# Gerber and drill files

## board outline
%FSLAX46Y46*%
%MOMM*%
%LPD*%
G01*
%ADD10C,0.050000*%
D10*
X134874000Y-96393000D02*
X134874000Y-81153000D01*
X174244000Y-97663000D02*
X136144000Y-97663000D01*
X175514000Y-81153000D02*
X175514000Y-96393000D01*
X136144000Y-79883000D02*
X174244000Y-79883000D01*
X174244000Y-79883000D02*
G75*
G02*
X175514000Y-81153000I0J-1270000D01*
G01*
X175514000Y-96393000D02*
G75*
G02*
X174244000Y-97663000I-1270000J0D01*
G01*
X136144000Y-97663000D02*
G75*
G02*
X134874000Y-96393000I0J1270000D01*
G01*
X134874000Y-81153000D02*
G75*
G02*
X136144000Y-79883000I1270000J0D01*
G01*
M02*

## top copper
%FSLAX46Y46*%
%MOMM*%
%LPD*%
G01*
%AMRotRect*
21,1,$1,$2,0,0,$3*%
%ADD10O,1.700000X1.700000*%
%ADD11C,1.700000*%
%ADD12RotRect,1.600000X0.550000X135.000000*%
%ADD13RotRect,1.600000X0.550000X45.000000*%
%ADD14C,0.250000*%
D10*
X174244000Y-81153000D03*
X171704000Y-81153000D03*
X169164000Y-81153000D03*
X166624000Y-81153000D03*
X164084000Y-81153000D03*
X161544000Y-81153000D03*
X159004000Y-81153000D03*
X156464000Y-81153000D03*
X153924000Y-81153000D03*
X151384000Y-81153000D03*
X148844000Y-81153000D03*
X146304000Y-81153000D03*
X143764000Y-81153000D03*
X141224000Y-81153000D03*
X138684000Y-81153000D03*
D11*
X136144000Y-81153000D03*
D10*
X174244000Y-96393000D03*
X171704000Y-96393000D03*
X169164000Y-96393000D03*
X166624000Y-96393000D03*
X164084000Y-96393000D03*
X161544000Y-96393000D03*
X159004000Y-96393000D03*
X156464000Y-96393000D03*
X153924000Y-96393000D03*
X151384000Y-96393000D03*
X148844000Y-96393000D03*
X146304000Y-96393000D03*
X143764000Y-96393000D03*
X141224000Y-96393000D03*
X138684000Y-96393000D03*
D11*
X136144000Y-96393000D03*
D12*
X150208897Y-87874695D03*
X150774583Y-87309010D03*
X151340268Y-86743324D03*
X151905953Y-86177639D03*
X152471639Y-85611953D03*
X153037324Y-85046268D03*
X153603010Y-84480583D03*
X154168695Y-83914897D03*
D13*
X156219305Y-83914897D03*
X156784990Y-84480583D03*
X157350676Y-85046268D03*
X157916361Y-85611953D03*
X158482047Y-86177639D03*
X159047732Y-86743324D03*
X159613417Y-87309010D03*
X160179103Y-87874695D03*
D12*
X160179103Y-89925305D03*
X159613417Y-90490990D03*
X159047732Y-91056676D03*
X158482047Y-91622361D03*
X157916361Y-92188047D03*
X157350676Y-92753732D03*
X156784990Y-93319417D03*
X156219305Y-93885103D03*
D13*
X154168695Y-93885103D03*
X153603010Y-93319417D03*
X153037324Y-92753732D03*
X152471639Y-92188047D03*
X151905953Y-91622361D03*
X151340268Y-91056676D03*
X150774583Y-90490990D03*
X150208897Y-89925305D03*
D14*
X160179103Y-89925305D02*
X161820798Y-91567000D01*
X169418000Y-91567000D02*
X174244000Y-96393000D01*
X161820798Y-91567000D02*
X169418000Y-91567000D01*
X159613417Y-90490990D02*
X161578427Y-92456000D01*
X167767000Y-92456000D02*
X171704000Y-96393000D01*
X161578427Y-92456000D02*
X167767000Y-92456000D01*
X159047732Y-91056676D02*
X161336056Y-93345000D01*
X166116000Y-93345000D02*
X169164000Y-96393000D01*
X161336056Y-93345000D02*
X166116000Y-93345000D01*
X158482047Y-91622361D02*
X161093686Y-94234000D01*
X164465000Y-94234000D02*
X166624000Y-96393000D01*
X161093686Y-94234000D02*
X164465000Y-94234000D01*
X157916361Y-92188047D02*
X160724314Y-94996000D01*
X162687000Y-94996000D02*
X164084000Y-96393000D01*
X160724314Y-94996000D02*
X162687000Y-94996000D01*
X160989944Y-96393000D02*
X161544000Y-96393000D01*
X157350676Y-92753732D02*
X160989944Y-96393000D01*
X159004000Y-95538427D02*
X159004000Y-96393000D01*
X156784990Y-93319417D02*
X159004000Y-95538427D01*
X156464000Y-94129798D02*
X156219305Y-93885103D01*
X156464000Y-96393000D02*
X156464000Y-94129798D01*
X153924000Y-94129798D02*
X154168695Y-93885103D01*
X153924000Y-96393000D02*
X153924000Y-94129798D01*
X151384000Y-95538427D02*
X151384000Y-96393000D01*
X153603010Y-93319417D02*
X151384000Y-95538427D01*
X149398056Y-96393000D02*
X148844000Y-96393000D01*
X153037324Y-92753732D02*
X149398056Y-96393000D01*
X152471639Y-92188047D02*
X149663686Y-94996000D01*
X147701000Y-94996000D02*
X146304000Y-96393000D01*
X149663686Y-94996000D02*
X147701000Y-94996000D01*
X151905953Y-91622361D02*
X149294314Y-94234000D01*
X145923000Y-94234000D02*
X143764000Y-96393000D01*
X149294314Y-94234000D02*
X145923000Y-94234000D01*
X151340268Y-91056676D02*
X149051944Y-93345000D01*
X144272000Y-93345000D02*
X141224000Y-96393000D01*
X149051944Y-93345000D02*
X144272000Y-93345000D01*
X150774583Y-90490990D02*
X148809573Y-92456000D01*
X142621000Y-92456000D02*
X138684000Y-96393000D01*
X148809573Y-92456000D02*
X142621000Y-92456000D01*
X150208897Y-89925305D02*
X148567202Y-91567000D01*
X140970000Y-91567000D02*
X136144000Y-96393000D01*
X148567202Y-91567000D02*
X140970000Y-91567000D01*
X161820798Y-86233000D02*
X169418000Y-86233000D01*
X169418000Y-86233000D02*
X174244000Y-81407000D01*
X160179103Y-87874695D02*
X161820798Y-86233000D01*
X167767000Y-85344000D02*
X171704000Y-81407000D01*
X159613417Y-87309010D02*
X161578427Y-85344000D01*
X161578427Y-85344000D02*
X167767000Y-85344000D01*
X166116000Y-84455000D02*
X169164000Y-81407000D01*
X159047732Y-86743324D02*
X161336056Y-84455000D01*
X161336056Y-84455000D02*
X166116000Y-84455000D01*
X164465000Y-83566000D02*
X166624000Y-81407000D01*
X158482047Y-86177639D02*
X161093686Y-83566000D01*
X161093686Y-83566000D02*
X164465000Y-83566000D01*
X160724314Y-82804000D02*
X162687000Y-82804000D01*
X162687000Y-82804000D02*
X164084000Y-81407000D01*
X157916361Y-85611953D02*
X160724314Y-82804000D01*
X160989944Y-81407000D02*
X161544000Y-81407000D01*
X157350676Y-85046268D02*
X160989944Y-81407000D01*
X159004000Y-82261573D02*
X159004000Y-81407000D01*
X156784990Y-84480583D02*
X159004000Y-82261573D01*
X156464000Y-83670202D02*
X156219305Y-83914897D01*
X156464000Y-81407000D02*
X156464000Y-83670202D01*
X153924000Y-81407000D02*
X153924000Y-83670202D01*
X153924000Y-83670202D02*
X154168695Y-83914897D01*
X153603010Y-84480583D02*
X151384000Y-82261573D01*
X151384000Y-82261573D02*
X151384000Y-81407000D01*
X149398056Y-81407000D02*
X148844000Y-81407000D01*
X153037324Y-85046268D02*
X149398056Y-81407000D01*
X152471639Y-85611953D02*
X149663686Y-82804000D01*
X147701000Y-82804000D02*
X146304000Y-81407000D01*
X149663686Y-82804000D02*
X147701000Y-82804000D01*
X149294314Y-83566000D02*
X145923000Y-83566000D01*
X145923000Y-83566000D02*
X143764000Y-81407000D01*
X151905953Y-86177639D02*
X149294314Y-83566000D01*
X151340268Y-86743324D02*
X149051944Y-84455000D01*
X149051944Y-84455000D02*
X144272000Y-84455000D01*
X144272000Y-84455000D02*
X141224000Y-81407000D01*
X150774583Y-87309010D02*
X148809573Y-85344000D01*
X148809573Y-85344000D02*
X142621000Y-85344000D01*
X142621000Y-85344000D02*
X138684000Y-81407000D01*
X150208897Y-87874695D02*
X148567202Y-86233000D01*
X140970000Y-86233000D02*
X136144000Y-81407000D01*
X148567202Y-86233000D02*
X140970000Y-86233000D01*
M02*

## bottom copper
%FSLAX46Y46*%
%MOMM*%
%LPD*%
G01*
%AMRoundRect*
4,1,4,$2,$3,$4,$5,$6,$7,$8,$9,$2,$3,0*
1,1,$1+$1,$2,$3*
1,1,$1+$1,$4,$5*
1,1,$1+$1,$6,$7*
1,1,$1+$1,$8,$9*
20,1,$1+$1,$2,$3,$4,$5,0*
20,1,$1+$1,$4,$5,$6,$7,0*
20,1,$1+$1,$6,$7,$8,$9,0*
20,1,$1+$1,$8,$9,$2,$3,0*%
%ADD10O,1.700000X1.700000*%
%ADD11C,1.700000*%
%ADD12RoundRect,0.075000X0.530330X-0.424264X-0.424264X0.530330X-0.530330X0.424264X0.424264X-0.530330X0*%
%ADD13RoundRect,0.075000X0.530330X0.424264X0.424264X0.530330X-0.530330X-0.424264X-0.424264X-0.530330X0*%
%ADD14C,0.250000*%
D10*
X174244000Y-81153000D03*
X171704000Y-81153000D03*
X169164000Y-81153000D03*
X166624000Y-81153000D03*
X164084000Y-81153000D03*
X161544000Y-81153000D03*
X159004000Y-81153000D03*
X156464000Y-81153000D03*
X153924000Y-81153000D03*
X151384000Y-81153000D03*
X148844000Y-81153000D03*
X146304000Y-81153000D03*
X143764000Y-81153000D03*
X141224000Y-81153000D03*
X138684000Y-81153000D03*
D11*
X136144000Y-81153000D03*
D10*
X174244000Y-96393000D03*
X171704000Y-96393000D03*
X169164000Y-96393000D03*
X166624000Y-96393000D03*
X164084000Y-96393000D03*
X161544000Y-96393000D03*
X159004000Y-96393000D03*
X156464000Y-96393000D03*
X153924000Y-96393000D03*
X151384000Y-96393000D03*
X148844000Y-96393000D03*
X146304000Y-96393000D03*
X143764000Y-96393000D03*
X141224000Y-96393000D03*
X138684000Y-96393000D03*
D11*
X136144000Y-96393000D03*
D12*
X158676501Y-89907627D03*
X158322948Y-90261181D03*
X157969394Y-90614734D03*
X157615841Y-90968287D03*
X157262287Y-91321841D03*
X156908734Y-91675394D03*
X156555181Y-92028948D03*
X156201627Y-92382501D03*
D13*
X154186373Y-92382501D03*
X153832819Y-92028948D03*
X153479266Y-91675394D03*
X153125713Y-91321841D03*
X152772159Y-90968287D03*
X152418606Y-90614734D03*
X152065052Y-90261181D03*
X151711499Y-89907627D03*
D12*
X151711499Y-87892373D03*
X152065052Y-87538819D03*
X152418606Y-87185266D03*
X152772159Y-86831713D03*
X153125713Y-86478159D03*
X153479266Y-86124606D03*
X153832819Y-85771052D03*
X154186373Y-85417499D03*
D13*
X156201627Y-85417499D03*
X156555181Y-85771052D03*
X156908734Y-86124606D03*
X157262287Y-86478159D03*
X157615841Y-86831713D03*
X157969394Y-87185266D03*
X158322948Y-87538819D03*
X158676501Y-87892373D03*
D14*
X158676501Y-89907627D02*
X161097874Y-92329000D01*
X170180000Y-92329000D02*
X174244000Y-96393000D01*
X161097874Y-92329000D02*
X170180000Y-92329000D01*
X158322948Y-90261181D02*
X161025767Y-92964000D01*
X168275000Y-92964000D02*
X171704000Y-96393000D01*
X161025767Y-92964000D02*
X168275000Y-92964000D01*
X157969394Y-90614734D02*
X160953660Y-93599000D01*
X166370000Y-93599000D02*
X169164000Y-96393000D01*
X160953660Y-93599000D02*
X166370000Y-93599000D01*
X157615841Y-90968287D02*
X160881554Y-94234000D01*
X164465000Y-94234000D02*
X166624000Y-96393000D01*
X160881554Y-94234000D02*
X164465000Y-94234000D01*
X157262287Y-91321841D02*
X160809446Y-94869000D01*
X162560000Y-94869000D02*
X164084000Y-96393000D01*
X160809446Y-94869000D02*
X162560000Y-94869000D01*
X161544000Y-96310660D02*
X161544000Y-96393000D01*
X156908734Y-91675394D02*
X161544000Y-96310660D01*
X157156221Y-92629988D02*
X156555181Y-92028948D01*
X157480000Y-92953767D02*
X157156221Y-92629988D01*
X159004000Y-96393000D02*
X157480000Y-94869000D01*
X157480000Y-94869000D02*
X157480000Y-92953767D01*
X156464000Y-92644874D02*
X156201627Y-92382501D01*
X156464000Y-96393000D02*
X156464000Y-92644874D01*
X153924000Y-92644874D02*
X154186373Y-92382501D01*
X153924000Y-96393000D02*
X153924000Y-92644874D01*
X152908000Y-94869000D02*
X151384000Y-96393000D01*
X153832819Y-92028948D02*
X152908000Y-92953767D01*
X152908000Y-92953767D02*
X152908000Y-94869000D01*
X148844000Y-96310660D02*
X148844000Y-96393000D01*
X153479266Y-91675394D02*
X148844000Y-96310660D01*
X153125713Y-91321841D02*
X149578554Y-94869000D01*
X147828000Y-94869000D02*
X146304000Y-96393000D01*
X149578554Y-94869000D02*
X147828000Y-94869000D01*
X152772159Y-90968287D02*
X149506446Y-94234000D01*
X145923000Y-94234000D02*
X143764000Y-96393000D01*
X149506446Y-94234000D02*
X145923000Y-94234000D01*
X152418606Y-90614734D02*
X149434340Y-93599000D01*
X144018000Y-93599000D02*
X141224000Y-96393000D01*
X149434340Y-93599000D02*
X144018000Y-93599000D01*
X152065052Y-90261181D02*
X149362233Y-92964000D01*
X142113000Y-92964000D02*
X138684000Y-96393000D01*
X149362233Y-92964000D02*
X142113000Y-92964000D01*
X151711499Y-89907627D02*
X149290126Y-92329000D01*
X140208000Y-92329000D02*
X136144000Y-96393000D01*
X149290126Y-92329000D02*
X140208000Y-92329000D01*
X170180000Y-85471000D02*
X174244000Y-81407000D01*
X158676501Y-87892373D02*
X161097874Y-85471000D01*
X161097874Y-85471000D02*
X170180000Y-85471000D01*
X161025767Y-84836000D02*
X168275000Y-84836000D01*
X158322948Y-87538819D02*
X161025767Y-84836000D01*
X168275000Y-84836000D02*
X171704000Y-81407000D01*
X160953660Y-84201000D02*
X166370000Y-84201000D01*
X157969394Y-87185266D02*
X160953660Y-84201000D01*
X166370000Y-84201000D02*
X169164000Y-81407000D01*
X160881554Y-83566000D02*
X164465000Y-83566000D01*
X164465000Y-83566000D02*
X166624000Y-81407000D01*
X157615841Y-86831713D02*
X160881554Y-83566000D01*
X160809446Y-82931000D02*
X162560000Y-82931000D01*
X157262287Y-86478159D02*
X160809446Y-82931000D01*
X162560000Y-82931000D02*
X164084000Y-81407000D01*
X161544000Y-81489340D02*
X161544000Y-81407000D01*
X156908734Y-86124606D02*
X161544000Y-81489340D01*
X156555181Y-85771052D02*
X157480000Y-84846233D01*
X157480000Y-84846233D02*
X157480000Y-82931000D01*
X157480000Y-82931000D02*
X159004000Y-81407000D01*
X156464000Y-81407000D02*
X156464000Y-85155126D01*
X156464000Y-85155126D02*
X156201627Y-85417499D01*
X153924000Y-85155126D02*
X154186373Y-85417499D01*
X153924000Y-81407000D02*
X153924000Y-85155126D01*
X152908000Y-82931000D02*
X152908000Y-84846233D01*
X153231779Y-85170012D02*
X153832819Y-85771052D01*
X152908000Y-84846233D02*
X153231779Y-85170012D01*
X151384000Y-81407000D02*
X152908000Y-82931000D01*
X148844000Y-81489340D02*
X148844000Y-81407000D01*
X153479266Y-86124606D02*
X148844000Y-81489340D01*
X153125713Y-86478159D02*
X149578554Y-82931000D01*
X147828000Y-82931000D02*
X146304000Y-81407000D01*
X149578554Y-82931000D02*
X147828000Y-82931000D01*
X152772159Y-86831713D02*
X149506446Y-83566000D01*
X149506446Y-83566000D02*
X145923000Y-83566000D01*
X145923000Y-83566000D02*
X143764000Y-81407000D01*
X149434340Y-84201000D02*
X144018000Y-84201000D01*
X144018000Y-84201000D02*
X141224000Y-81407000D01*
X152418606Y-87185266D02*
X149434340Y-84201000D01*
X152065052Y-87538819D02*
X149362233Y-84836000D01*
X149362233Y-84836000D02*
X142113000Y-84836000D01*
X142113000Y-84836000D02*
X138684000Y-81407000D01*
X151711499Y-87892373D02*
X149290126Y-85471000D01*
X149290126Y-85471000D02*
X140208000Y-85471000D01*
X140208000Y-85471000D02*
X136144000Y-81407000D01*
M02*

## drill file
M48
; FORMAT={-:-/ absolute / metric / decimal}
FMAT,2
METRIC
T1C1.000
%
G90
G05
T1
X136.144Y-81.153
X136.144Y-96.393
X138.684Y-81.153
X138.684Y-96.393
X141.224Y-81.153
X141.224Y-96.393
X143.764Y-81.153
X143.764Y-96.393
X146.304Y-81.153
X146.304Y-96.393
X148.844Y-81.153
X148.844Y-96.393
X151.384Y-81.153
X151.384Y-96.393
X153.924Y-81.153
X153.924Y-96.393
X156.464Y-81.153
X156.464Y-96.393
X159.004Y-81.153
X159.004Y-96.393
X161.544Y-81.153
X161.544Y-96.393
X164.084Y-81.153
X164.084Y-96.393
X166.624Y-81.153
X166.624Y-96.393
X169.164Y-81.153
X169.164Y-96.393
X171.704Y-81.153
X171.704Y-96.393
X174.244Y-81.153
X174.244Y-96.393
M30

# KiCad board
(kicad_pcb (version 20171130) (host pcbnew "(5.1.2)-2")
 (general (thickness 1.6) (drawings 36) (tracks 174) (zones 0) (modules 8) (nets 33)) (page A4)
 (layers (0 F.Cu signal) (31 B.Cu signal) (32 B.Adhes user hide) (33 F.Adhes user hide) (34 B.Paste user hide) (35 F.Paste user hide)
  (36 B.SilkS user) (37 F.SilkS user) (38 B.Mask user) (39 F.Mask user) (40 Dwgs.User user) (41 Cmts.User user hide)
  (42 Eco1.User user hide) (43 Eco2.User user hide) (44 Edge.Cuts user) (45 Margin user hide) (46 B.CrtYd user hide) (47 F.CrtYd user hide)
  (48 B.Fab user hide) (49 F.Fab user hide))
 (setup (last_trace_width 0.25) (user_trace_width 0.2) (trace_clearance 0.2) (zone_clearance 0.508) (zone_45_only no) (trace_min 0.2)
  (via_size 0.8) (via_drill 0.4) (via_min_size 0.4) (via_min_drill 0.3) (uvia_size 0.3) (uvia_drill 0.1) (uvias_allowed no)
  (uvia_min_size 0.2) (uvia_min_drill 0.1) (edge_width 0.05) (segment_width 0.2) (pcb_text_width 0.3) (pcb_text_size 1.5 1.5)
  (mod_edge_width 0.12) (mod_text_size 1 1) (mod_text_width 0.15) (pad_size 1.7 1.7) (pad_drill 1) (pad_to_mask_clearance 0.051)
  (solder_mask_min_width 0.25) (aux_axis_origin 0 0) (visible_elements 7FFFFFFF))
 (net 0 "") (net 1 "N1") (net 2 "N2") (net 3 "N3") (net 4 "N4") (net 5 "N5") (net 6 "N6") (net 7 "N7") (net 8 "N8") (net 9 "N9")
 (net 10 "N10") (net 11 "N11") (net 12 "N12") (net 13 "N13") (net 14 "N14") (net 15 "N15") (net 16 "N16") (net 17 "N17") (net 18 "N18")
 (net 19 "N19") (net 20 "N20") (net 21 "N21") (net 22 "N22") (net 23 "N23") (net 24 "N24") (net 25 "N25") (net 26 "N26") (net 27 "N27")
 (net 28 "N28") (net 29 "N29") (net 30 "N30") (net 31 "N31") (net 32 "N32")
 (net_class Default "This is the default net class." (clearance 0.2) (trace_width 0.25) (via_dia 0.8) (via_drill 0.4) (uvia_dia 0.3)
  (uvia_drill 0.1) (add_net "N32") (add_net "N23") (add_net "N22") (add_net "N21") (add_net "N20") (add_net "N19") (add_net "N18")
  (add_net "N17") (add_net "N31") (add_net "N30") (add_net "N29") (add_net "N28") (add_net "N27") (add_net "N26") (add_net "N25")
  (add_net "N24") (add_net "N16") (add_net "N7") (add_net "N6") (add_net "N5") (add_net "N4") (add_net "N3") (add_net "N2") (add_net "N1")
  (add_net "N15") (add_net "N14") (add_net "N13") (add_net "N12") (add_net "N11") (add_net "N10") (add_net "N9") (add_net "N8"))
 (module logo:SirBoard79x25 (layer B.Cu) (at 169.164 93.599 180)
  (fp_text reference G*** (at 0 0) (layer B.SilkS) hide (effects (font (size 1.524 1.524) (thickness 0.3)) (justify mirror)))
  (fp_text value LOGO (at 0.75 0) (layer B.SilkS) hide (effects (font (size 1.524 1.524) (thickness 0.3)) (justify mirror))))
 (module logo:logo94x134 (layer B.Cu) (at 169.164 87.122 180)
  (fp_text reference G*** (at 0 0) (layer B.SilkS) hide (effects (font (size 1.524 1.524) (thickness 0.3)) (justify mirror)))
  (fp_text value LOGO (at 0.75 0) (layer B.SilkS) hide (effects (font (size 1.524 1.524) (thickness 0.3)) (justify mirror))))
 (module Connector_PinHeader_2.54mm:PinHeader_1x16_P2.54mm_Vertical (layer B.Cu) (at 136.144 81.153 270)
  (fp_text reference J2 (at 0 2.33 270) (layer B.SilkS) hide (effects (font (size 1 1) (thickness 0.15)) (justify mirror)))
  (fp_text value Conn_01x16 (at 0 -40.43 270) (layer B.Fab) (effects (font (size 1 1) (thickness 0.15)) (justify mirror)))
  (pad 16 thru_hole oval (at 0 -38.1 270) (size 1.7 1.7) (drill 1) (layers *.Cu *.Mask) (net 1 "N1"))
  (pad 15 thru_hole oval (at 0 -35.56 270) (size 1.7 1.7) (drill 1) (layers *.Cu *.Mask) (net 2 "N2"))
  (pad 14 thru_hole oval (at 0 -33.02 270) (size 1.7 1.7) (drill 1) (layers *.Cu *.Mask) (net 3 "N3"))
  (pad 13 thru_hole oval (at 0 -30.48 270) (size 1.7 1.7) (drill 1) (layers *.Cu *.Mask) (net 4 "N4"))
  (pad 12 thru_hole oval (at 0 -27.94 270) (size 1.7 1.7) (drill 1) (layers *.Cu *.Mask) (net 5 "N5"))
  (pad 11 thru_hole oval (at 0 -25.4 270) (size 1.7 1.7) (drill 1) (layers *.Cu *.Mask) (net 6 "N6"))
  (pad 10 thru_hole oval (at 0 -22.86 270) (size 1.7 1.7) (drill 1) (layers *.Cu *.Mask) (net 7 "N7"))
  (pad 9 thru_hole oval (at 0 -20.32 270) (size 1.7 1.7) (drill 1) (layers *.Cu *.Mask) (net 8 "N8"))
  (pad 8 thru_hole oval (at 0 -17.78 270) (size 1.7 1.7) (drill 1) (layers *.Cu *.Mask) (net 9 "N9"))
  (pad 7 thru_hole oval (at 0 -15.24 270) (size 1.7 1.7) (drill 1) (layers *.Cu *.Mask) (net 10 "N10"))
  (pad 6 thru_hole oval (at 0 -12.7 270) (size 1.7 1.7) (drill 1) (layers *.Cu *.Mask) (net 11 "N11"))
  (pad 5 thru_hole oval (at 0 -10.16 270) (size 1.7 1.7) (drill 1) (layers *.Cu *.Mask) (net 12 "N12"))
  (pad 4 thru_hole oval (at 0 -7.62 270) (size 1.7 1.7) (drill 1) (layers *.Cu *.Mask) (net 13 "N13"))
  (pad 3 thru_hole oval (at 0 -5.08 270) (size 1.7 1.7) (drill 1) (layers *.Cu *.Mask) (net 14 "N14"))
  (pad 2 thru_hole oval (at 0 -2.54 270) (size 1.7 1.7) (drill 1) (layers *.Cu *.Mask) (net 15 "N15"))
  (pad 1 thru_hole circle (at 0 0 270) (size 1.7 1.7) (drill 1) (layers *.Cu *.Mask) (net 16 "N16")))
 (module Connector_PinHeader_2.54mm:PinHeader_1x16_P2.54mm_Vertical (layer B.Cu) (at 136.144 96.393 270)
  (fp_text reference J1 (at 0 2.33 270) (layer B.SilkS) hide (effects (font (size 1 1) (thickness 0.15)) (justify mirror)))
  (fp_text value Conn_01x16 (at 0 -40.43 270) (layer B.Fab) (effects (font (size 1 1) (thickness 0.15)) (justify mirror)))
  (pad 16 thru_hole oval (at 0 -38.1 270) (size 1.7 1.7) (drill 1) (layers *.Cu *.Mask) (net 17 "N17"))
  (pad 15 thru_hole oval (at 0 -35.56 270) (size 1.7 1.7) (drill 1) (layers *.Cu *.Mask) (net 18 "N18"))
  (pad 14 thru_hole oval (at 0 -33.02 270) (size 1.7 1.7) (drill 1) (layers *.Cu *.Mask) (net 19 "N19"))
  (pad 13 thru_hole oval (at 0 -30.48 270) (size 1.7 1.7) (drill 1) (layers *.Cu *.Mask) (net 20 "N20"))
  (pad 12 thru_hole oval (at 0 -27.94 270) (size 1.7 1.7) (drill 1) (layers *.Cu *.Mask) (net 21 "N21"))
  (pad 11 thru_hole oval (at 0 -25.4 270) (size 1.7 1.7) (drill 1) (layers *.Cu *.Mask) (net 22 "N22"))
  (pad 10 thru_hole oval (at 0 -22.86 270) (size 1.7 1.7) (drill 1) (layers *.Cu *.Mask) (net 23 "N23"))
  (pad 9 thru_hole oval (at 0 -20.32 270) (size 1.7 1.7) (drill 1) (layers *.Cu *.Mask) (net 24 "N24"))
  (pad 8 thru_hole oval (at 0 -17.78 270) (size 1.7 1.7) (drill 1) (layers *.Cu *.Mask) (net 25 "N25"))
  (pad 7 thru_hole oval (at 0 -15.24 270) (size 1.7 1.7) (drill 1) (layers *.Cu *.Mask) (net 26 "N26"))
  (pad 6 thru_hole oval (at 0 -12.7 270) (size 1.7 1.7) (drill 1) (layers *.Cu *.Mask) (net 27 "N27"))
  (pad 5 thru_hole oval (at 0 -10.16 270) (size 1.7 1.7) (drill 1) (layers *.Cu *.Mask) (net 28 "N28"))
  (pad 4 thru_hole oval (at 0 -7.62 270) (size 1.7 1.7) (drill 1) (layers *.Cu *.Mask) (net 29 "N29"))
  (pad 3 thru_hole oval (at 0 -5.08 270) (size 1.7 1.7) (drill 1) (layers *.Cu *.Mask) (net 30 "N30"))
  (pad 2 thru_hole oval (at 0 -2.54 270) (size 1.7 1.7) (drill 1) (layers *.Cu *.Mask) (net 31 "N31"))
  (pad 1 thru_hole circle (at 0 0 270) (size 1.7 1.7) (drill 1) (layers *.Cu *.Mask) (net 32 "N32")))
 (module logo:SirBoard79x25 (layer F.Cu) (at 141.224 93.726)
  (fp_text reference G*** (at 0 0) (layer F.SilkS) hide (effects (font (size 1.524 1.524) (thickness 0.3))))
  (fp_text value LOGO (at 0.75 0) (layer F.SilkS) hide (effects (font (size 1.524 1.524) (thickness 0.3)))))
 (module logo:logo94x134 (layer F.Cu) (at 141.224 87.249)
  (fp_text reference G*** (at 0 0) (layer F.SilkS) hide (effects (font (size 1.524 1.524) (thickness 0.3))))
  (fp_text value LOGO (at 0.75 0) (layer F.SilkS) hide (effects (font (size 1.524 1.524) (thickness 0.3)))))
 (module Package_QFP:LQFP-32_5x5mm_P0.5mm (layer B.Cu) (at 155.194 88.9 135)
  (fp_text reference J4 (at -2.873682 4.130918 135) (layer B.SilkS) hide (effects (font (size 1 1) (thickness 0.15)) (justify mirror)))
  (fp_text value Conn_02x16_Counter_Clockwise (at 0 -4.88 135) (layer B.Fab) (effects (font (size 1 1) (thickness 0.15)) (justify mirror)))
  (pad 1 smd roundrect (at -3.175 1.75 135) (size 1.5 0.3) (layers B.Cu B.Paste B.Mask) (roundrect_rratio 0.25) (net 17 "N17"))
  (pad 2 smd roundrect (at -3.175 1.25 135) (size 1.5 0.3) (layers B.Cu B.Paste B.Mask) (roundrect_rratio 0.25) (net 18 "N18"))
  (pad 3 smd roundrect (at -3.175 0.75 135) (size 1.5 0.3) (layers B.Cu B.Paste B.Mask) (roundrect_rratio 0.25) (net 19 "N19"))
  (pad 4 smd roundrect (at -3.175 0.25 135) (size 1.5 0.3) (layers B.Cu B.Paste B.Mask) (roundrect_rratio 0.25) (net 20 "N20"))
  (pad 5 smd roundrect (at -3.175 -0.25 135) (size 1.5 0.3) (layers B.Cu B.Paste B.Mask) (roundrect_rratio 0.25) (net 21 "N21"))
  (pad 6 smd roundrect (at -3.175 -0.75 135) (size 1.5 0.3) (layers B.Cu B.Paste B.Mask) (roundrect_rratio 0.25) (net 22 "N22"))
  (pad 7 smd roundrect (at -3.175 -1.25 135) (size 1.5 0.3) (layers B.Cu B.Paste B.Mask) (roundrect_rratio 0.25) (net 23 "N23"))
  (pad 8 smd roundrect (at -3.175 -1.75 135) (size 1.5 0.3) (layers B.Cu B.Paste B.Mask) (roundrect_rratio 0.25) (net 24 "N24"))
  (pad 9 smd roundrect (at -1.75 -3.175 135) (size 0.3 1.5) (layers B.Cu B.Paste B.Mask) (roundrect_rratio 0.25) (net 25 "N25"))
  (pad 10 smd roundrect (at -1.25 -3.175 135) (size 0.3 1.5) (layers B.Cu B.Paste B.Mask) (roundrect_rratio 0.25) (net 26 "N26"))
  (pad 11 smd roundrect (at -0.75 -3.175 135) (size 0.3 1.5) (layers B.Cu B.Paste B.Mask) (roundrect_rratio 0.25) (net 27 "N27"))
  (pad 12 smd roundrect (at -0.25 -3.175 135) (size 0.3 1.5) (layers B.Cu B.Paste B.Mask) (roundrect_rratio 0.25) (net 28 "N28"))
  (pad 13 smd roundrect (at 0.25 -3.175 135) (size 0.3 1.5) (layers B.Cu B.Paste B.Mask) (roundrect_rratio 0.25) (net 29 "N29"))
  (pad 14 smd roundrect (at 0.75 -3.175 135) (size 0.3 1.5) (layers B.Cu B.Paste B.Mask) (roundrect_rratio 0.25) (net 30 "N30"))
  (pad 15 smd roundrect (at 1.25 -3.175 135) (size 0.3 1.5) (layers B.Cu B.Paste B.Mask) (roundrect_rratio 0.25) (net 31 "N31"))
  (pad 16 smd roundrect (at 1.75 -3.175 135) (size 0.3 1.5) (layers B.Cu B.Paste B.Mask) (roundrect_rratio 0.25) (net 32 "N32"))
  (pad 17 smd roundrect (at 3.175 -1.75 135) (size 1.5 0.3) (layers B.Cu B.Paste B.Mask) (roundrect_rratio 0.25) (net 16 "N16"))
  (pad 18 smd roundrect (at 3.175 -1.25 135) (size 1.5 0.3) (layers B.Cu B.Paste B.Mask) (roundrect_rratio 0.25) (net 15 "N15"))
  (pad 19 smd roundrect (at 3.175 -0.75 135) (size 1.5 0.3) (layers B.Cu B.Paste B.Mask) (roundrect_rratio 0.25) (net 14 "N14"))
  (pad 20 smd roundrect (at 3.175 -0.25 135) (size 1.5 0.3) (layers B.Cu B.Paste B.Mask) (roundrect_rratio 0.25) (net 13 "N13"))
  (pad 21 smd roundrect (at 3.175 0.25 135) (size 1.5 0.3) (layers B.Cu B.Paste B.Mask) (roundrect_rratio 0.25) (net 12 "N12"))
  (pad 22 smd roundrect (at 3.175 0.75 135) (size 1.5 0.3) (layers B.Cu B.Paste B.Mask) (roundrect_rratio 0.25) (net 11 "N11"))
  (pad 23 smd roundrect (at 3.175 1.25 135) (size 1.5 0.3) (layers B.Cu B.Paste B.Mask) (roundrect_rratio 0.25) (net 10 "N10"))
  (pad 24 smd roundrect (at 3.175 1.75 135) (size 1.5 0.3) (layers B.Cu B.Paste B.Mask) (roundrect_rratio 0.25) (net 9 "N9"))
  (pad 25 smd roundrect (at 1.75 3.175 135) (size 0.3 1.5) (layers B.Cu B.Paste B.Mask) (roundrect_rratio 0.25) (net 8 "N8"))
  (pad 26 smd roundrect (at 1.25 3.175 135) (size 0.3 1.5) (layers B.Cu B.Paste B.Mask) (roundrect_rratio 0.25) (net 7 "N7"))
  (pad 27 smd roundrect (at 0.75 3.175 135) (size 0.3 1.5) (layers B.Cu B.Paste B.Mask) (roundrect_rratio 0.25) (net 6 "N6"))
  (pad 28 smd roundrect (at 0.25 3.175 135) (size 0.3 1.5) (layers B.Cu B.Paste B.Mask) (roundrect_rratio 0.25) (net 5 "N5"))
  (pad 29 smd roundrect (at -0.25 3.175 135) (size 0.3 1.5) (layers B.Cu B.Paste B.Mask) (roundrect_rratio 0.25) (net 4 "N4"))
  (pad 30 smd roundrect (at -0.75 3.175 135) (size 0.3 1.5) (layers B.Cu B.Paste B.Mask) (roundrect_rratio 0.25) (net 3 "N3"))
  (pad 31 smd roundrect (at -1.25 3.175 135) (size 0.3 1.5) (layers B.Cu B.Paste B.Mask) (roundrect_rratio 0.25) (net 2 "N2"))
  (pad 32 smd roundrect (at -1.75 3.175 135) (size 0.3 1.5) (layers B.Cu B.Paste B.Mask) (roundrect_rratio 0.25) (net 1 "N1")))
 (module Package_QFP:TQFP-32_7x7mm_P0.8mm (layer F.Cu) (at 155.194 88.9 45)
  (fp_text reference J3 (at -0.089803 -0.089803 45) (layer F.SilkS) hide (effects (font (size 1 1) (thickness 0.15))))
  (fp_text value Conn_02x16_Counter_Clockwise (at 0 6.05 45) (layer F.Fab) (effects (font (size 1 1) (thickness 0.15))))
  (pad 32 smd rect (at -2.8 -4.25 135) (size 1.6 0.55) (layers F.Cu F.Paste F.Mask) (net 16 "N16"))
  (pad 31 smd rect (at -2 -4.25 135) (size 1.6 0.55) (layers F.Cu F.Paste F.Mask) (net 15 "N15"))
  (pad 30 smd rect (at -1.2 -4.25 135) (size 1.6 0.55) (layers F.Cu F.Paste F.Mask) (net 14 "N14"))
  (pad 29 smd rect (at -0.4 -4.25 135) (size 1.6 0.55) (layers F.Cu F.Paste F.Mask) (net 13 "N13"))
  (pad 28 smd rect (at 0.4 -4.25 135) (size 1.6 0.55) (layers F.Cu F.Paste F.Mask) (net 12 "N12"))
  (pad 27 smd rect (at 1.2 -4.25 135) (size 1.6 0.55) (layers F.Cu F.Paste F.Mask) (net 11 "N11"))
  (pad 26 smd rect (at 2 -4.25 135) (size 1.6 0.55) (layers F.Cu F.Paste F.Mask) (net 10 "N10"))
  (pad 25 smd rect (at 2.8 -4.25 135) (size 1.6 0.55) (layers F.Cu F.Paste F.Mask) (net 9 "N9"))
  (pad 24 smd rect (at 4.25 -2.8 45) (size 1.6 0.55) (layers F.Cu F.Paste F.Mask) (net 8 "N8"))
  (pad 23 smd rect (at 4.25 -2 45) (size 1.6 0.55) (layers F.Cu F.Paste F.Mask) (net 7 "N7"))
  (pad 22 smd rect (at 4.25 -1.2 45) (size 1.6 0.55) (layers F.Cu F.Paste F.Mask) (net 6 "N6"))
  (pad 21 smd rect (at 4.25 -0.4 45) (size 1.6 0.55) (layers F.Cu F.Paste F.Mask) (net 5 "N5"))
  (pad 20 smd rect (at 4.25 0.4 45) (size 1.6 0.55) (layers F.Cu F.Paste F.Mask) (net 4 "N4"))
  (pad 19 smd rect (at 4.25 1.2 45) (size 1.6 0.55) (layers F.Cu F.Paste F.Mask) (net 3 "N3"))
  (pad 18 smd rect (at 4.25 2 45) (size 1.6 0.55) (layers F.Cu F.Paste F.Mask) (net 2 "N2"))
  (pad 17 smd rect (at 4.25 2.8 45) (size 1.6 0.55) (layers F.Cu F.Paste F.Mask) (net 1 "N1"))
  (pad 16 smd rect (at 2.8 4.25 135) (size 1.6 0.55) (layers F.Cu F.Paste F.Mask) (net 17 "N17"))
  (pad 15 smd rect (at 2 4.25 135) (size 1.6 0.55) (layers F.Cu F.Paste F.Mask) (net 18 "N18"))
  (pad 14 smd rect (at 1.2 4.25 135) (size 1.6 0.55) (layers F.Cu F.Paste F.Mask) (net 19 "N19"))
  (pad 13 smd rect (at 0.4 4.25 135) (size 1.6 0.55) (layers F.Cu F.Paste F.Mask) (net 20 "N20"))
  (pad 12 smd rect (at -0.4 4.25 135) (size 1.6 0.55) (layers F.Cu F.Paste F.Mask) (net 21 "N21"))
  (pad 11 smd rect (at -1.2 4.25 135) (size 1.6 0.55) (layers F.Cu F.Paste F.Mask) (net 22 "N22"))
  (pad 10 smd rect (at -2 4.25 135) (size 1.6 0.55) (layers F.Cu F.Paste F.Mask) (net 23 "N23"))
  (pad 9 smd rect (at -2.8 4.25 135) (size 1.6 0.55) (layers F.Cu F.Paste F.Mask) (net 24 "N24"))
  (pad 8 smd rect (at -4.25 2.8 45) (size 1.6 0.55) (layers F.Cu F.Paste F.Mask) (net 25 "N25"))
  (pad 7 smd rect (at -4.25 2 45) (size 1.6 0.55) (layers F.Cu F.Paste F.Mask) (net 26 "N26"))
  (pad 6 smd rect (at -4.25 1.2 45) (size 1.6 0.55) (layers F.Cu F.Paste F.Mask) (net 27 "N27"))
  (pad 5 smd rect (at -4.25 0.4 45) (size 1.6 0.55) (layers F.Cu F.Paste F.Mask) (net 28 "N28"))
  (pad 4 smd rect (at -4.25 -0.4 45) (size 1.6 0.55) (layers F.Cu F.Paste F.Mask) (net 29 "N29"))
  (pad 3 smd rect (at -4.25 -1.2 45) (size 1.6 0.55) (layers F.Cu F.Paste F.Mask) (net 30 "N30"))
  (pad 2 smd rect (at -4.25 -2 45) (size 1.6 0.55) (layers F.Cu F.Paste F.Mask) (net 31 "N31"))
  (pad 1 smd rect (at -4.25 -2.8 45) (size 1.6 0.55) (layers F.Cu F.Paste F.Mask) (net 32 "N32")))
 (gr_line (start 134.874 96.393) (end 134.874 81.153) (layer Edge.Cuts) (width 0.05))
 (gr_line (start 174.244 97.663) (end 136.144 97.663) (layer Edge.Cuts) (width 0.05))
 (gr_line (start 175.514 81.153) (end 175.514 96.393) (layer Edge.Cuts) (width 0.05))
 (gr_line (start 136.144 79.883) (end 174.244 79.883) (layer Edge.Cuts) (width 0.05))
 (gr_arc (start 174.244 81.153) (end 175.514 81.153) (angle -90) (layer Edge.Cuts) (width 0.05))
 (gr_arc (start 174.244 96.393) (end 174.244 97.663) (angle -90) (layer Edge.Cuts) (width 0.05))
 (gr_arc (start 136.144 96.393) (end 134.874 96.393) (angle -90) (layer Edge.Cuts) (width 0.05))
 (gr_arc (start 136.144 81.153) (end 136.144 79.883) (angle -90) (layer Edge.Cuts) (width 0.05))
 (segment (start 160.179103 89.925305) (end 161.820798 91.567) (width 0.25) (layer F.Cu) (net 17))
 (segment (start 169.418 91.567) (end 174.244 96.393) (width 0.25) (layer F.Cu) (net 17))
 (segment (start 161.820798 91.567) (end 169.418 91.567) (width 0.25) (layer F.Cu) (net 17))
 (segment (start 158.676501 89.907627) (end 161.097874 92.329) (width 0.25) (layer B.Cu) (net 17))
 (segment (start 170.18 92.329) (end 174.244 96.393) (width 0.25) (layer B.Cu) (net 17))
 (segment (start 161.097874 92.329) (end 170.18 92.329) (width 0.25) (layer B.Cu) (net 17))
 (segment (start 159.613417 90.49099) (end 161.578427 92.456) (width 0.25) (layer F.Cu) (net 18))
 (segment (start 167.767 92.456) (end 171.704 96.393) (width 0.25) (layer F.Cu) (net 18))
 (segment (start 161.578427 92.456) (end 167.767 92.456) (width 0.25) (layer F.Cu) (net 18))
 (segment (start 158.322948 90.261181) (end 161.025767 92.964) (width 0.25) (layer B.Cu) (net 18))
 (segment (start 168.275 92.964) (end 171.704 96.393) (width 0.25) (layer B.Cu) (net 18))
 (segment (start 161.025767 92.964) (end 168.275 92.964) (width 0.25) (layer B.Cu) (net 18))
 (segment (start 159.047732 91.056676) (end 161.336056 93.345) (width 0.25) (layer F.Cu) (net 19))
 (segment (start 166.116 93.345) (end 169.164 96.393) (width 0.25) (layer F.Cu) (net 19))
 (segment (start 161.336056 93.345) (end 166.116 93.345) (width 0.25) (layer F.Cu) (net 19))
 (segment (start 157.969394 90.614734) (end 160.95366 93.599) (width 0.25) (layer B.Cu) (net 19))
 (segment (start 166.37 93.599) (end 169.164 96.393) (width 0.25) (layer B.Cu) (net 19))
 (segment (start 160.95366 93.599) (end 166.37 93.599) (width 0.25) (layer B.Cu) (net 19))
 (segment (start 158.482047 91.622361) (end 161.093686 94.234) (width 0.25) (layer F.Cu) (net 20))
 (segment (start 164.465 94.234) (end 166.624 96.393) (width 0.25) (layer F.Cu) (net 20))
 (segment (start 161.093686 94.234) (end 164.465 94.234) (width 0.25) (layer F.Cu) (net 20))
 (segment (start 157.615841 90.968287) (end 160.881554 94.234) (width 0.25) (layer B.Cu) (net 20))
 (segment (start 164.465 94.234) (end 166.624 96.393) (width 0.25) (layer B.Cu) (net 20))
 (segment (start 160.881554 94.234) (end 164.465 94.234) (width 0.25) (layer B.Cu) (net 20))
 (segment (start 157.916361 92.188047) (end 160.724314 94.996) (width 0.25) (layer F.Cu) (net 21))
 (segment (start 162.687 94.996) (end 164.084 96.393) (width 0.25) (layer F.Cu) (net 21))
 (segment (start 160.724314 94.996) (end 162.687 94.996) (width 0.25) (layer F.Cu) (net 21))
 (segment (start 157.262287 91.321841) (end 160.809446 94.869) (width 0.25) (layer B.Cu) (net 21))
 (segment (start 162.56 94.869) (end 164.084 96.393) (width 0.25) (layer B.Cu) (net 21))
 (segment (start 160.809446 94.869) (end 162.56 94.869) (width 0.25) (layer B.Cu) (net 21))
 (segment (start 160.989944 96.393) (end 161.544 96.393) (width 0.25) (layer F.Cu) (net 22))
 (segment (start 157.350676 92.753732) (end 160.989944 96.393) (width 0.25) (layer F.Cu) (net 22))
 (segment (start 161.544 96.31066) (end 161.544 96.393) (width 0.25) (layer B.Cu) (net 22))
 (segment (start 156.908734 91.675394) (end 161.544 96.31066) (width 0.25) (layer B.Cu) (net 22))
 (segment (start 159.004 95.538427) (end 159.004 96.393) (width 0.25) (layer F.Cu) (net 23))
 (segment (start 156.78499 93.319417) (end 159.004 95.538427) (width 0.25) (layer F.Cu) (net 23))
 (segment (start 157.156221 92.629988) (end 156.555181 92.028948) (width 0.25) (layer B.Cu) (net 23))
 (segment (start 157.48 92.953767) (end 157.156221 92.629988) (width 0.25) (layer B.Cu) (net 23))
 (segment (start 159.004 96.393) (end 157.48 94.869) (width 0.25) (layer B.Cu) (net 23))
 (segment (start 157.48 94.869) (end 157.48 92.953767) (width 0.25) (layer B.Cu) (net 23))
 (segment (start 156.464 94.129798) (end 156.219305 93.885103) (width 0.25) (layer F.Cu) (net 24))
 (segment (start 156.464 96.393) (end 156.464 94.129798) (width 0.25) (layer F.Cu) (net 24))
 (segment (start 156.464 92.644874) (end 156.201627 92.382501) (width 0.25) (layer B.Cu) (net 24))
 (segment (start 156.464 96.393) (end 156.464 92.644874) (width 0.25) (layer B.Cu) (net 24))
 (segment (start 153.924 94.129798) (end 154.168695 93.885103) (width 0.25) (layer F.Cu) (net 25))
 (segment (start 153.924 96.393) (end 153.924 94.129798) (width 0.25) (layer F.Cu) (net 25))
 (segment (start 153.924 92.644874) (end 154.186373 92.382501) (width 0.25) (layer B.Cu) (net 25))
 (segment (start 153.924 96.393) (end 153.924 92.644874) (width 0.25) (layer B.Cu) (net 25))
 (segment (start 151.384 95.538427) (end 151.384 96.393) (width 0.25) (layer F.Cu) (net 26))
 (segment (start 153.60301 93.319417) (end 151.384 95.538427) (width 0.25) (layer F.Cu) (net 26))
 (segment (start 152.908 94.869) (end 151.384 96.393) (width 0.25) (layer B.Cu) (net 26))
 (segment (start 153.832819 92.028948) (end 152.908 92.953767) (width 0.25) (layer B.Cu) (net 26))
 (segment (start 152.908 92.953767) (end 152.908 94.869) (width 0.25) (layer B.Cu) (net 26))
 (segment (start 149.398056 96.393) (end 148.844 96.393) (width 0.25) (layer F.Cu) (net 27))
 (segment (start 153.037324 92.753732) (end 149.398056 96.393) (width 0.25) (layer F.Cu) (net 27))
 (segment (start 148.844 96.31066) (end 148.844 96.393) (width 0.25) (layer B.Cu) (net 27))
 (segment (start 153.479266 91.675394) (end 148.844 96.31066) (width 0.25) (layer B.Cu) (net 27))
 (segment (start 152.471639 92.188047) (end 149.663686 94.996) (width 0.25) (layer F.Cu) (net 28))
 (segment (start 147.701 94.996) (end 146.304 96.393) (width 0.25) (layer F.Cu) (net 28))
 (segment (start 149.663686 94.996) (end 147.701 94.996) (width 0.25) (layer F.Cu) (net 28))
 (segment (start 153.125713 91.321841) (end 149.578554 94.869) (width 0.25) (layer B.Cu) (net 28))
 (segment (start 147.828 94.869) (end 146.304 96.393) (width 0.25) (layer B.Cu) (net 28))
 (segment (start 149.578554 94.869) (end 147.828 94.869) (width 0.25) (layer B.Cu) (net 28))
 (segment (start 151.905953 91.622361) (end 149.294314 94.234) (width 0.25) (layer F.Cu) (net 29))
 (segment (start 145.923 94.234) (end 143.764 96.393) (width 0.25) (layer F.Cu) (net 29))
 (segment (start 149.294314 94.234) (end 145.923 94.234) (width 0.25) (layer F.Cu) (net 29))
 (segment (start 152.772159 90.968287) (end 149.506446 94.234) (width 0.25) (layer B.Cu) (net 29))
 (segment (start 145.923 94.234) (end 143.764 96.393) (width 0.25) (layer B.Cu) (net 29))
 (segment (start 149.506446 94.234) (end 145.923 94.234) (width 0.25) (layer B.Cu) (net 29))
 (segment (start 151.340268 91.056676) (end 149.051944 93.345) (width 0.25) (layer F.Cu) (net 30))
 (segment (start 144.272 93.345) (end 141.224 96.393) (width 0.25) (layer F.Cu) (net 30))
 (segment (start 149.051944 93.345) (end 144.272 93.345) (width 0.25) (layer F.Cu) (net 30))
 (segment (start 152.418606 90.614734) (end 149.43434 93.599) (width 0.25) (layer B.Cu) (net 30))
 (segment (start 144.018 93.599) (end 141.224 96.393) (width 0.25) (layer B.Cu) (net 30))
 (segment (start 149.43434 93.599) (end 144.018 93.599) (width 0.25) (layer B.Cu) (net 30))
 (segment (start 150.774583 90.49099) (end 148.809573 92.456) (width 0.25) (layer F.Cu) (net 31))
 (segment (start 142.621 92.456) (end 138.684 96.393) (width 0.25) (layer F.Cu) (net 31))
 (segment (start 148.809573 92.456) (end 142.621 92.456) (width 0.25) (layer F.Cu) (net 31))
 (segment (start 152.065052 90.261181) (end 149.362233 92.964) (width 0.25) (layer B.Cu) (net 31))
 (segment (start 142.113 92.964) (end 138.684 96.393) (width 0.25) (layer B.Cu) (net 31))
 (segment (start 149.362233 92.964) (end 142.113 92.964) (width 0.25) (layer B.Cu) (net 31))
 (segment (start 150.208897 89.925305) (end 148.567202 91.567) (width 0.25) (layer F.Cu) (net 32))
 (segment (start 140.97 91.567) (end 136.144 96.393) (width 0.25) (layer F.Cu) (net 32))
 (segment (start 148.567202 91.567) (end 140.97 91.567) (width 0.25) (layer F.Cu) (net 32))
 (segment (start 151.711499 89.907627) (end 149.290126 92.329) (width 0.25) (layer B.Cu) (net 32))
 (segment (start 140.208 92.329) (end 136.144 96.393) (width 0.25) (layer B.Cu) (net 32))
 (segment (start 149.290126 92.329) (end 140.208 92.329) (width 0.25) (layer B.Cu) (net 32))
 (segment (start 170.18 85.471) (end 174.244 81.407) (width 0.25) (layer B.Cu) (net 1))
 (segment (start 158.676501 87.892373) (end 161.097874 85.471) (width 0.25) (layer B.Cu) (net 1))
 (segment (start 161.820798 86.233) (end 169.418 86.233) (width 0.25) (layer F.Cu) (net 1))
 (segment (start 169.418 86.233) (end 174.244 81.407) (width 0.25) (layer F.Cu) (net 1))
 (segment (start 160.179103 87.874695) (end 161.820798 86.233) (width 0.25) (layer F.Cu) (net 1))
 (segment (start 161.097874 85.471) (end 170.18 85.471) (width 0.25) (layer B.Cu) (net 1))
 (segment (start 167.767 85.344) (end 171.704 81.407) (width 0.25) (layer F.Cu) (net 2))
 (segment (start 161.025767 84.836) (end 168.275 84.836) (width 0.25) (layer B.Cu) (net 2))
 (segment (start 159.613417 87.30901) (end 161.578427 85.344) (width 0.25) (layer F.Cu) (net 2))
 (segment (start 161.578427 85.344) (end 167.767 85.344) (width 0.25) (layer F.Cu) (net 2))
 (segment (start 158.322948 87.538819) (end 161.025767 84.836) (width 0.25) (layer B.Cu) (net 2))
 (segment (start 168.275 84.836) (end 171.704 81.407) (width 0.25) (layer B.Cu) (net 2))
 (segment (start 160.95366 84.201) (end 166.37 84.201) (width 0.25) (layer B.Cu) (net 3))
 (segment (start 157.969394 87.185266) (end 160.95366 84.201) (width 0.25) (layer B.Cu) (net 3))
 (segment (start 166.37 84.201) (end 169.164 81.407) (width 0.25) (layer B.Cu) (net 3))
 (segment (start 166.116 84.455) (end 169.164 81.407) (width 0.25) (layer F.Cu) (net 3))
 (segment (start 159.047732 86.743324) (end 161.336056 84.455) (width 0.25) (layer F.Cu) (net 3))
 (segment (start 161.336056 84.455) (end 166.116 84.455) (width 0.25) (layer F.Cu) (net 3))
 (segment (start 164.465 83.566) (end 166.624 81.407) (width 0.25) (layer F.Cu) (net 4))
 (segment (start 158.482047 86.177639) (end 161.093686 83.566) (width 0.25) (layer F.Cu) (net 4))
 (segment (start 161.093686 83.566) (end 164.465 83.566) (width 0.25) (layer F.Cu) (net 4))
 (segment (start 160.881554 83.566) (end 164.465 83.566) (width 0.25) (layer B.Cu) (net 4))
 (segment (start 164.465 83.566) (end 166.624 81.407) (width 0.25) (layer B.Cu) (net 4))
 (segment (start 157.615841 86.831713) (end 160.881554 83.566) (width 0.25) (layer B.Cu) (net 4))
 (segment (start 160.724314 82.804) (end 162.687 82.804) (width 0.25) (layer F.Cu) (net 5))
 (segment (start 162.687 82.804) (end 164.084 81.407) (width 0.25) (layer F.Cu) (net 5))
 (segment (start 157.916361 85.611953) (end 160.724314 82.804) (width 0.25) (layer F.Cu) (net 5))
 (segment (start 160.809446 82.931) (end 162.56 82.931) (width 0.25) (layer B.Cu) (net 5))
 (segment (start 157.262287 86.478159) (end 160.809446 82.931) (width 0.25) (layer B.Cu) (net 5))
 (segment (start 162.56 82.931) (end 164.084 81.407) (width 0.25) (layer B.Cu) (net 5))
 (segment (start 160.989944 81.407) (end 161.544 81.407) (width 0.25) (layer F.Cu) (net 6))
 (segment (start 157.350676 85.046268) (end 160.989944 81.407) (width 0.25) (layer F.Cu) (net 6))
 (segment (start 161.544 81.48934) (end 161.544 81.407) (width 0.25) (layer B.Cu) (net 6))
 (segment (start 156.908734 86.124606) (end 161.544 81.48934) (width 0.25) (layer B.Cu) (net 6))
 (segment (start 159.004 82.261573) (end 159.004 81.407) (width 0.25) (layer F.Cu) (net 7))
 (segment (start 156.78499 84.480583) (end 159.004 82.261573) (width 0.25) (layer F.Cu) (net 7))
 (segment (start 156.555181 85.771052) (end 157.48 84.846233) (width 0.25) (layer B.Cu) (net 7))
 (segment (start 157.48 84.846233) (end 157.48 82.931) (width 0.25) (layer B.Cu) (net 7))
 (segment (start 157.48 82.931) (end 159.004 81.407) (width 0.25) (layer B.Cu) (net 7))
 (segment (start 156.464 83.670202) (end 156.219305 83.914897) (width 0.25) (layer F.Cu) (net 8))
 (segment (start 156.464 81.407) (end 156.464 83.670202) (width 0.25) (layer F.Cu) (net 8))
 (segment (start 156.464 81.407) (end 156.464 85.155126) (width 0.25) (layer B.Cu) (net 8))
 (segment (start 156.464 85.155126) (end 156.201627 85.417499) (width 0.25) (layer B.Cu) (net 8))
 (segment (start 153.924 81.407) (end 153.924 83.670202) (width 0.25) (layer F.Cu) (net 9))
 (segment (start 153.924 83.670202) (end 154.168695 83.914897) (width 0.25) (layer F.Cu) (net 9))
 (segment (start 153.924 85.155126) (end 154.186373 85.417499) (width 0.25) (layer B.Cu) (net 9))
 (segment (start 153.924 81.407) (end 153.924 85.155126) (width 0.25) (layer B.Cu) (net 9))
 (segment (start 153.60301 84.480583) (end 151.384 82.261573) (width 0.25) (layer F.Cu) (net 10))
 (segment (start 151.384 82.261573) (end 151.384 81.407) (width 0.25) (layer F.Cu) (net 10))
 (segment (start 152.908 82.931) (end 152.908 84.846233) (width 0.25) (layer B.Cu) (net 10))
 (segment (start 153.231779 85.170012) (end 153.832819 85.771052) (width 0.25) (layer B.Cu) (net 10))
 (segment (start 152.908 84.846233) (end 153.231779 85.170012) (width 0.25) (layer B.Cu) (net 10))
 (segment (start 151.384 81.407) (end 152.908 82.931) (width 0.25) (layer B.Cu) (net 10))
 (segment (start 149.398056 81.407) (end 148.844 81.407) (width 0.25) (layer F.Cu) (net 11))
 (segment (start 153.037324 85.046268) (end 149.398056 81.407) (width 0.25) (layer F.Cu) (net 11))
 (segment (start 148.844 81.48934) (end 148.844 81.407) (width 0.25) (layer B.Cu) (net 11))
 (segment (start 153.479266 86.124606) (end 148.844 81.48934) (width 0.25) (layer B.Cu) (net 11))
 (segment (start 152.471639 85.611953) (end 149.663686 82.804) (width 0.25) (layer F.Cu) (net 12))
 (segment (start 147.701 82.804) (end 146.304 81.407) (width 0.25) (layer F.Cu) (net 12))
 (segment (start 149.663686 82.804) (end 147.701 82.804) (width 0.25) (layer F.Cu) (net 12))
 (segment (start 153.125713 86.478159) (end 149.578554 82.931) (width 0.25) (layer B.Cu) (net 12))
 (segment (start 147.828 82.931) (end 146.304 81.407) (width 0.25) (layer B.Cu) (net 12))
 (segment (start 149.578554 82.931) (end 147.828 82.931) (width 0.25) (layer B.Cu) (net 12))
 (segment (start 149.294314 83.566) (end 145.923 83.566) (width 0.25) (layer F.Cu) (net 13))
 (segment (start 145.923 83.566) (end 143.764 81.407) (width 0.25) (layer F.Cu) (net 13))
 (segment (start 151.905953 86.177639) (end 149.294314 83.566) (width 0.25) (layer F.Cu) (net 13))
 (segment (start 152.772159 86.831713) (end 149.506446 83.566) (width 0.25) (layer B.Cu) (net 13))
 (segment (start 149.506446 83.566) (end 145.923 83.566) (width 0.25) (layer B.Cu) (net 13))
 (segment (start 145.923 83.566) (end 143.764 81.407) (width 0.25) (layer B.Cu) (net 13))
 (segment (start 151.340268 86.743324) (end 149.051944 84.455) (width 0.25) (layer F.Cu) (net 14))
 (segment (start 149.051944 84.455) (end 144.272 84.455) (width 0.25) (layer F.Cu) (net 14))
 (segment (start 144.272 84.455) (end 141.224 81.407) (width 0.25) (layer F.Cu) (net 14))
 (segment (start 149.43434 84.201) (end 144.018 84.201) (width 0.25) (layer B.Cu) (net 14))
 (segment (start 144.018 84.201) (end 141.224 81.407) (width 0.25) (layer B.Cu) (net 14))
 (segment (start 152.418606 87.185266) (end 149.43434 84.201) (width 0.25) (layer B.Cu) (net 14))
 (segment (start 150.774583 87.30901) (end 148.809573 85.344) (width 0.25) (layer F.Cu) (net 15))
 (segment (start 148.809573 85.344) (end 142.621 85.344) (width 0.25) (layer F.Cu) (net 15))
 (segment (start 142.621 85.344) (end 138.684 81.407) (width 0.25) (layer F.Cu) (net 15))
 (segment (start 152.065052 87.538819) (end 149.362233 84.836) (width 0.25) (layer B.Cu) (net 15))
 (segment (start 149.362233 84.836) (end 142.113 84.836) (width 0.25) (layer B.Cu) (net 15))
 (segment (start 142.113 84.836) (end 138.684 81.407) (width 0.25) (layer B.Cu) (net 15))
 (segment (start 150.208897 87.874695) (end 148.567202 86.233) (width 0.25) (layer F.Cu) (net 16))
 (segment (start 140.97 86.233) (end 136.144 81.407) (width 0.25) (layer F.Cu) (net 16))
 (segment (start 148.567202 86.233) (end 140.97 86.233) (width 0.25) (layer F.Cu) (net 16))
 (segment (start 151.711499 87.892373) (end 149.290126 85.471) (width 0.25) (layer B.Cu) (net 16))
 (segment (start 149.290126 85.471) (end 140.208 85.471) (width 0.25) (layer B.Cu) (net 16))
 (segment (start 140.208 85.471) (end 136.144 81.407) (width 0.25) (layer B.Cu) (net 16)))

